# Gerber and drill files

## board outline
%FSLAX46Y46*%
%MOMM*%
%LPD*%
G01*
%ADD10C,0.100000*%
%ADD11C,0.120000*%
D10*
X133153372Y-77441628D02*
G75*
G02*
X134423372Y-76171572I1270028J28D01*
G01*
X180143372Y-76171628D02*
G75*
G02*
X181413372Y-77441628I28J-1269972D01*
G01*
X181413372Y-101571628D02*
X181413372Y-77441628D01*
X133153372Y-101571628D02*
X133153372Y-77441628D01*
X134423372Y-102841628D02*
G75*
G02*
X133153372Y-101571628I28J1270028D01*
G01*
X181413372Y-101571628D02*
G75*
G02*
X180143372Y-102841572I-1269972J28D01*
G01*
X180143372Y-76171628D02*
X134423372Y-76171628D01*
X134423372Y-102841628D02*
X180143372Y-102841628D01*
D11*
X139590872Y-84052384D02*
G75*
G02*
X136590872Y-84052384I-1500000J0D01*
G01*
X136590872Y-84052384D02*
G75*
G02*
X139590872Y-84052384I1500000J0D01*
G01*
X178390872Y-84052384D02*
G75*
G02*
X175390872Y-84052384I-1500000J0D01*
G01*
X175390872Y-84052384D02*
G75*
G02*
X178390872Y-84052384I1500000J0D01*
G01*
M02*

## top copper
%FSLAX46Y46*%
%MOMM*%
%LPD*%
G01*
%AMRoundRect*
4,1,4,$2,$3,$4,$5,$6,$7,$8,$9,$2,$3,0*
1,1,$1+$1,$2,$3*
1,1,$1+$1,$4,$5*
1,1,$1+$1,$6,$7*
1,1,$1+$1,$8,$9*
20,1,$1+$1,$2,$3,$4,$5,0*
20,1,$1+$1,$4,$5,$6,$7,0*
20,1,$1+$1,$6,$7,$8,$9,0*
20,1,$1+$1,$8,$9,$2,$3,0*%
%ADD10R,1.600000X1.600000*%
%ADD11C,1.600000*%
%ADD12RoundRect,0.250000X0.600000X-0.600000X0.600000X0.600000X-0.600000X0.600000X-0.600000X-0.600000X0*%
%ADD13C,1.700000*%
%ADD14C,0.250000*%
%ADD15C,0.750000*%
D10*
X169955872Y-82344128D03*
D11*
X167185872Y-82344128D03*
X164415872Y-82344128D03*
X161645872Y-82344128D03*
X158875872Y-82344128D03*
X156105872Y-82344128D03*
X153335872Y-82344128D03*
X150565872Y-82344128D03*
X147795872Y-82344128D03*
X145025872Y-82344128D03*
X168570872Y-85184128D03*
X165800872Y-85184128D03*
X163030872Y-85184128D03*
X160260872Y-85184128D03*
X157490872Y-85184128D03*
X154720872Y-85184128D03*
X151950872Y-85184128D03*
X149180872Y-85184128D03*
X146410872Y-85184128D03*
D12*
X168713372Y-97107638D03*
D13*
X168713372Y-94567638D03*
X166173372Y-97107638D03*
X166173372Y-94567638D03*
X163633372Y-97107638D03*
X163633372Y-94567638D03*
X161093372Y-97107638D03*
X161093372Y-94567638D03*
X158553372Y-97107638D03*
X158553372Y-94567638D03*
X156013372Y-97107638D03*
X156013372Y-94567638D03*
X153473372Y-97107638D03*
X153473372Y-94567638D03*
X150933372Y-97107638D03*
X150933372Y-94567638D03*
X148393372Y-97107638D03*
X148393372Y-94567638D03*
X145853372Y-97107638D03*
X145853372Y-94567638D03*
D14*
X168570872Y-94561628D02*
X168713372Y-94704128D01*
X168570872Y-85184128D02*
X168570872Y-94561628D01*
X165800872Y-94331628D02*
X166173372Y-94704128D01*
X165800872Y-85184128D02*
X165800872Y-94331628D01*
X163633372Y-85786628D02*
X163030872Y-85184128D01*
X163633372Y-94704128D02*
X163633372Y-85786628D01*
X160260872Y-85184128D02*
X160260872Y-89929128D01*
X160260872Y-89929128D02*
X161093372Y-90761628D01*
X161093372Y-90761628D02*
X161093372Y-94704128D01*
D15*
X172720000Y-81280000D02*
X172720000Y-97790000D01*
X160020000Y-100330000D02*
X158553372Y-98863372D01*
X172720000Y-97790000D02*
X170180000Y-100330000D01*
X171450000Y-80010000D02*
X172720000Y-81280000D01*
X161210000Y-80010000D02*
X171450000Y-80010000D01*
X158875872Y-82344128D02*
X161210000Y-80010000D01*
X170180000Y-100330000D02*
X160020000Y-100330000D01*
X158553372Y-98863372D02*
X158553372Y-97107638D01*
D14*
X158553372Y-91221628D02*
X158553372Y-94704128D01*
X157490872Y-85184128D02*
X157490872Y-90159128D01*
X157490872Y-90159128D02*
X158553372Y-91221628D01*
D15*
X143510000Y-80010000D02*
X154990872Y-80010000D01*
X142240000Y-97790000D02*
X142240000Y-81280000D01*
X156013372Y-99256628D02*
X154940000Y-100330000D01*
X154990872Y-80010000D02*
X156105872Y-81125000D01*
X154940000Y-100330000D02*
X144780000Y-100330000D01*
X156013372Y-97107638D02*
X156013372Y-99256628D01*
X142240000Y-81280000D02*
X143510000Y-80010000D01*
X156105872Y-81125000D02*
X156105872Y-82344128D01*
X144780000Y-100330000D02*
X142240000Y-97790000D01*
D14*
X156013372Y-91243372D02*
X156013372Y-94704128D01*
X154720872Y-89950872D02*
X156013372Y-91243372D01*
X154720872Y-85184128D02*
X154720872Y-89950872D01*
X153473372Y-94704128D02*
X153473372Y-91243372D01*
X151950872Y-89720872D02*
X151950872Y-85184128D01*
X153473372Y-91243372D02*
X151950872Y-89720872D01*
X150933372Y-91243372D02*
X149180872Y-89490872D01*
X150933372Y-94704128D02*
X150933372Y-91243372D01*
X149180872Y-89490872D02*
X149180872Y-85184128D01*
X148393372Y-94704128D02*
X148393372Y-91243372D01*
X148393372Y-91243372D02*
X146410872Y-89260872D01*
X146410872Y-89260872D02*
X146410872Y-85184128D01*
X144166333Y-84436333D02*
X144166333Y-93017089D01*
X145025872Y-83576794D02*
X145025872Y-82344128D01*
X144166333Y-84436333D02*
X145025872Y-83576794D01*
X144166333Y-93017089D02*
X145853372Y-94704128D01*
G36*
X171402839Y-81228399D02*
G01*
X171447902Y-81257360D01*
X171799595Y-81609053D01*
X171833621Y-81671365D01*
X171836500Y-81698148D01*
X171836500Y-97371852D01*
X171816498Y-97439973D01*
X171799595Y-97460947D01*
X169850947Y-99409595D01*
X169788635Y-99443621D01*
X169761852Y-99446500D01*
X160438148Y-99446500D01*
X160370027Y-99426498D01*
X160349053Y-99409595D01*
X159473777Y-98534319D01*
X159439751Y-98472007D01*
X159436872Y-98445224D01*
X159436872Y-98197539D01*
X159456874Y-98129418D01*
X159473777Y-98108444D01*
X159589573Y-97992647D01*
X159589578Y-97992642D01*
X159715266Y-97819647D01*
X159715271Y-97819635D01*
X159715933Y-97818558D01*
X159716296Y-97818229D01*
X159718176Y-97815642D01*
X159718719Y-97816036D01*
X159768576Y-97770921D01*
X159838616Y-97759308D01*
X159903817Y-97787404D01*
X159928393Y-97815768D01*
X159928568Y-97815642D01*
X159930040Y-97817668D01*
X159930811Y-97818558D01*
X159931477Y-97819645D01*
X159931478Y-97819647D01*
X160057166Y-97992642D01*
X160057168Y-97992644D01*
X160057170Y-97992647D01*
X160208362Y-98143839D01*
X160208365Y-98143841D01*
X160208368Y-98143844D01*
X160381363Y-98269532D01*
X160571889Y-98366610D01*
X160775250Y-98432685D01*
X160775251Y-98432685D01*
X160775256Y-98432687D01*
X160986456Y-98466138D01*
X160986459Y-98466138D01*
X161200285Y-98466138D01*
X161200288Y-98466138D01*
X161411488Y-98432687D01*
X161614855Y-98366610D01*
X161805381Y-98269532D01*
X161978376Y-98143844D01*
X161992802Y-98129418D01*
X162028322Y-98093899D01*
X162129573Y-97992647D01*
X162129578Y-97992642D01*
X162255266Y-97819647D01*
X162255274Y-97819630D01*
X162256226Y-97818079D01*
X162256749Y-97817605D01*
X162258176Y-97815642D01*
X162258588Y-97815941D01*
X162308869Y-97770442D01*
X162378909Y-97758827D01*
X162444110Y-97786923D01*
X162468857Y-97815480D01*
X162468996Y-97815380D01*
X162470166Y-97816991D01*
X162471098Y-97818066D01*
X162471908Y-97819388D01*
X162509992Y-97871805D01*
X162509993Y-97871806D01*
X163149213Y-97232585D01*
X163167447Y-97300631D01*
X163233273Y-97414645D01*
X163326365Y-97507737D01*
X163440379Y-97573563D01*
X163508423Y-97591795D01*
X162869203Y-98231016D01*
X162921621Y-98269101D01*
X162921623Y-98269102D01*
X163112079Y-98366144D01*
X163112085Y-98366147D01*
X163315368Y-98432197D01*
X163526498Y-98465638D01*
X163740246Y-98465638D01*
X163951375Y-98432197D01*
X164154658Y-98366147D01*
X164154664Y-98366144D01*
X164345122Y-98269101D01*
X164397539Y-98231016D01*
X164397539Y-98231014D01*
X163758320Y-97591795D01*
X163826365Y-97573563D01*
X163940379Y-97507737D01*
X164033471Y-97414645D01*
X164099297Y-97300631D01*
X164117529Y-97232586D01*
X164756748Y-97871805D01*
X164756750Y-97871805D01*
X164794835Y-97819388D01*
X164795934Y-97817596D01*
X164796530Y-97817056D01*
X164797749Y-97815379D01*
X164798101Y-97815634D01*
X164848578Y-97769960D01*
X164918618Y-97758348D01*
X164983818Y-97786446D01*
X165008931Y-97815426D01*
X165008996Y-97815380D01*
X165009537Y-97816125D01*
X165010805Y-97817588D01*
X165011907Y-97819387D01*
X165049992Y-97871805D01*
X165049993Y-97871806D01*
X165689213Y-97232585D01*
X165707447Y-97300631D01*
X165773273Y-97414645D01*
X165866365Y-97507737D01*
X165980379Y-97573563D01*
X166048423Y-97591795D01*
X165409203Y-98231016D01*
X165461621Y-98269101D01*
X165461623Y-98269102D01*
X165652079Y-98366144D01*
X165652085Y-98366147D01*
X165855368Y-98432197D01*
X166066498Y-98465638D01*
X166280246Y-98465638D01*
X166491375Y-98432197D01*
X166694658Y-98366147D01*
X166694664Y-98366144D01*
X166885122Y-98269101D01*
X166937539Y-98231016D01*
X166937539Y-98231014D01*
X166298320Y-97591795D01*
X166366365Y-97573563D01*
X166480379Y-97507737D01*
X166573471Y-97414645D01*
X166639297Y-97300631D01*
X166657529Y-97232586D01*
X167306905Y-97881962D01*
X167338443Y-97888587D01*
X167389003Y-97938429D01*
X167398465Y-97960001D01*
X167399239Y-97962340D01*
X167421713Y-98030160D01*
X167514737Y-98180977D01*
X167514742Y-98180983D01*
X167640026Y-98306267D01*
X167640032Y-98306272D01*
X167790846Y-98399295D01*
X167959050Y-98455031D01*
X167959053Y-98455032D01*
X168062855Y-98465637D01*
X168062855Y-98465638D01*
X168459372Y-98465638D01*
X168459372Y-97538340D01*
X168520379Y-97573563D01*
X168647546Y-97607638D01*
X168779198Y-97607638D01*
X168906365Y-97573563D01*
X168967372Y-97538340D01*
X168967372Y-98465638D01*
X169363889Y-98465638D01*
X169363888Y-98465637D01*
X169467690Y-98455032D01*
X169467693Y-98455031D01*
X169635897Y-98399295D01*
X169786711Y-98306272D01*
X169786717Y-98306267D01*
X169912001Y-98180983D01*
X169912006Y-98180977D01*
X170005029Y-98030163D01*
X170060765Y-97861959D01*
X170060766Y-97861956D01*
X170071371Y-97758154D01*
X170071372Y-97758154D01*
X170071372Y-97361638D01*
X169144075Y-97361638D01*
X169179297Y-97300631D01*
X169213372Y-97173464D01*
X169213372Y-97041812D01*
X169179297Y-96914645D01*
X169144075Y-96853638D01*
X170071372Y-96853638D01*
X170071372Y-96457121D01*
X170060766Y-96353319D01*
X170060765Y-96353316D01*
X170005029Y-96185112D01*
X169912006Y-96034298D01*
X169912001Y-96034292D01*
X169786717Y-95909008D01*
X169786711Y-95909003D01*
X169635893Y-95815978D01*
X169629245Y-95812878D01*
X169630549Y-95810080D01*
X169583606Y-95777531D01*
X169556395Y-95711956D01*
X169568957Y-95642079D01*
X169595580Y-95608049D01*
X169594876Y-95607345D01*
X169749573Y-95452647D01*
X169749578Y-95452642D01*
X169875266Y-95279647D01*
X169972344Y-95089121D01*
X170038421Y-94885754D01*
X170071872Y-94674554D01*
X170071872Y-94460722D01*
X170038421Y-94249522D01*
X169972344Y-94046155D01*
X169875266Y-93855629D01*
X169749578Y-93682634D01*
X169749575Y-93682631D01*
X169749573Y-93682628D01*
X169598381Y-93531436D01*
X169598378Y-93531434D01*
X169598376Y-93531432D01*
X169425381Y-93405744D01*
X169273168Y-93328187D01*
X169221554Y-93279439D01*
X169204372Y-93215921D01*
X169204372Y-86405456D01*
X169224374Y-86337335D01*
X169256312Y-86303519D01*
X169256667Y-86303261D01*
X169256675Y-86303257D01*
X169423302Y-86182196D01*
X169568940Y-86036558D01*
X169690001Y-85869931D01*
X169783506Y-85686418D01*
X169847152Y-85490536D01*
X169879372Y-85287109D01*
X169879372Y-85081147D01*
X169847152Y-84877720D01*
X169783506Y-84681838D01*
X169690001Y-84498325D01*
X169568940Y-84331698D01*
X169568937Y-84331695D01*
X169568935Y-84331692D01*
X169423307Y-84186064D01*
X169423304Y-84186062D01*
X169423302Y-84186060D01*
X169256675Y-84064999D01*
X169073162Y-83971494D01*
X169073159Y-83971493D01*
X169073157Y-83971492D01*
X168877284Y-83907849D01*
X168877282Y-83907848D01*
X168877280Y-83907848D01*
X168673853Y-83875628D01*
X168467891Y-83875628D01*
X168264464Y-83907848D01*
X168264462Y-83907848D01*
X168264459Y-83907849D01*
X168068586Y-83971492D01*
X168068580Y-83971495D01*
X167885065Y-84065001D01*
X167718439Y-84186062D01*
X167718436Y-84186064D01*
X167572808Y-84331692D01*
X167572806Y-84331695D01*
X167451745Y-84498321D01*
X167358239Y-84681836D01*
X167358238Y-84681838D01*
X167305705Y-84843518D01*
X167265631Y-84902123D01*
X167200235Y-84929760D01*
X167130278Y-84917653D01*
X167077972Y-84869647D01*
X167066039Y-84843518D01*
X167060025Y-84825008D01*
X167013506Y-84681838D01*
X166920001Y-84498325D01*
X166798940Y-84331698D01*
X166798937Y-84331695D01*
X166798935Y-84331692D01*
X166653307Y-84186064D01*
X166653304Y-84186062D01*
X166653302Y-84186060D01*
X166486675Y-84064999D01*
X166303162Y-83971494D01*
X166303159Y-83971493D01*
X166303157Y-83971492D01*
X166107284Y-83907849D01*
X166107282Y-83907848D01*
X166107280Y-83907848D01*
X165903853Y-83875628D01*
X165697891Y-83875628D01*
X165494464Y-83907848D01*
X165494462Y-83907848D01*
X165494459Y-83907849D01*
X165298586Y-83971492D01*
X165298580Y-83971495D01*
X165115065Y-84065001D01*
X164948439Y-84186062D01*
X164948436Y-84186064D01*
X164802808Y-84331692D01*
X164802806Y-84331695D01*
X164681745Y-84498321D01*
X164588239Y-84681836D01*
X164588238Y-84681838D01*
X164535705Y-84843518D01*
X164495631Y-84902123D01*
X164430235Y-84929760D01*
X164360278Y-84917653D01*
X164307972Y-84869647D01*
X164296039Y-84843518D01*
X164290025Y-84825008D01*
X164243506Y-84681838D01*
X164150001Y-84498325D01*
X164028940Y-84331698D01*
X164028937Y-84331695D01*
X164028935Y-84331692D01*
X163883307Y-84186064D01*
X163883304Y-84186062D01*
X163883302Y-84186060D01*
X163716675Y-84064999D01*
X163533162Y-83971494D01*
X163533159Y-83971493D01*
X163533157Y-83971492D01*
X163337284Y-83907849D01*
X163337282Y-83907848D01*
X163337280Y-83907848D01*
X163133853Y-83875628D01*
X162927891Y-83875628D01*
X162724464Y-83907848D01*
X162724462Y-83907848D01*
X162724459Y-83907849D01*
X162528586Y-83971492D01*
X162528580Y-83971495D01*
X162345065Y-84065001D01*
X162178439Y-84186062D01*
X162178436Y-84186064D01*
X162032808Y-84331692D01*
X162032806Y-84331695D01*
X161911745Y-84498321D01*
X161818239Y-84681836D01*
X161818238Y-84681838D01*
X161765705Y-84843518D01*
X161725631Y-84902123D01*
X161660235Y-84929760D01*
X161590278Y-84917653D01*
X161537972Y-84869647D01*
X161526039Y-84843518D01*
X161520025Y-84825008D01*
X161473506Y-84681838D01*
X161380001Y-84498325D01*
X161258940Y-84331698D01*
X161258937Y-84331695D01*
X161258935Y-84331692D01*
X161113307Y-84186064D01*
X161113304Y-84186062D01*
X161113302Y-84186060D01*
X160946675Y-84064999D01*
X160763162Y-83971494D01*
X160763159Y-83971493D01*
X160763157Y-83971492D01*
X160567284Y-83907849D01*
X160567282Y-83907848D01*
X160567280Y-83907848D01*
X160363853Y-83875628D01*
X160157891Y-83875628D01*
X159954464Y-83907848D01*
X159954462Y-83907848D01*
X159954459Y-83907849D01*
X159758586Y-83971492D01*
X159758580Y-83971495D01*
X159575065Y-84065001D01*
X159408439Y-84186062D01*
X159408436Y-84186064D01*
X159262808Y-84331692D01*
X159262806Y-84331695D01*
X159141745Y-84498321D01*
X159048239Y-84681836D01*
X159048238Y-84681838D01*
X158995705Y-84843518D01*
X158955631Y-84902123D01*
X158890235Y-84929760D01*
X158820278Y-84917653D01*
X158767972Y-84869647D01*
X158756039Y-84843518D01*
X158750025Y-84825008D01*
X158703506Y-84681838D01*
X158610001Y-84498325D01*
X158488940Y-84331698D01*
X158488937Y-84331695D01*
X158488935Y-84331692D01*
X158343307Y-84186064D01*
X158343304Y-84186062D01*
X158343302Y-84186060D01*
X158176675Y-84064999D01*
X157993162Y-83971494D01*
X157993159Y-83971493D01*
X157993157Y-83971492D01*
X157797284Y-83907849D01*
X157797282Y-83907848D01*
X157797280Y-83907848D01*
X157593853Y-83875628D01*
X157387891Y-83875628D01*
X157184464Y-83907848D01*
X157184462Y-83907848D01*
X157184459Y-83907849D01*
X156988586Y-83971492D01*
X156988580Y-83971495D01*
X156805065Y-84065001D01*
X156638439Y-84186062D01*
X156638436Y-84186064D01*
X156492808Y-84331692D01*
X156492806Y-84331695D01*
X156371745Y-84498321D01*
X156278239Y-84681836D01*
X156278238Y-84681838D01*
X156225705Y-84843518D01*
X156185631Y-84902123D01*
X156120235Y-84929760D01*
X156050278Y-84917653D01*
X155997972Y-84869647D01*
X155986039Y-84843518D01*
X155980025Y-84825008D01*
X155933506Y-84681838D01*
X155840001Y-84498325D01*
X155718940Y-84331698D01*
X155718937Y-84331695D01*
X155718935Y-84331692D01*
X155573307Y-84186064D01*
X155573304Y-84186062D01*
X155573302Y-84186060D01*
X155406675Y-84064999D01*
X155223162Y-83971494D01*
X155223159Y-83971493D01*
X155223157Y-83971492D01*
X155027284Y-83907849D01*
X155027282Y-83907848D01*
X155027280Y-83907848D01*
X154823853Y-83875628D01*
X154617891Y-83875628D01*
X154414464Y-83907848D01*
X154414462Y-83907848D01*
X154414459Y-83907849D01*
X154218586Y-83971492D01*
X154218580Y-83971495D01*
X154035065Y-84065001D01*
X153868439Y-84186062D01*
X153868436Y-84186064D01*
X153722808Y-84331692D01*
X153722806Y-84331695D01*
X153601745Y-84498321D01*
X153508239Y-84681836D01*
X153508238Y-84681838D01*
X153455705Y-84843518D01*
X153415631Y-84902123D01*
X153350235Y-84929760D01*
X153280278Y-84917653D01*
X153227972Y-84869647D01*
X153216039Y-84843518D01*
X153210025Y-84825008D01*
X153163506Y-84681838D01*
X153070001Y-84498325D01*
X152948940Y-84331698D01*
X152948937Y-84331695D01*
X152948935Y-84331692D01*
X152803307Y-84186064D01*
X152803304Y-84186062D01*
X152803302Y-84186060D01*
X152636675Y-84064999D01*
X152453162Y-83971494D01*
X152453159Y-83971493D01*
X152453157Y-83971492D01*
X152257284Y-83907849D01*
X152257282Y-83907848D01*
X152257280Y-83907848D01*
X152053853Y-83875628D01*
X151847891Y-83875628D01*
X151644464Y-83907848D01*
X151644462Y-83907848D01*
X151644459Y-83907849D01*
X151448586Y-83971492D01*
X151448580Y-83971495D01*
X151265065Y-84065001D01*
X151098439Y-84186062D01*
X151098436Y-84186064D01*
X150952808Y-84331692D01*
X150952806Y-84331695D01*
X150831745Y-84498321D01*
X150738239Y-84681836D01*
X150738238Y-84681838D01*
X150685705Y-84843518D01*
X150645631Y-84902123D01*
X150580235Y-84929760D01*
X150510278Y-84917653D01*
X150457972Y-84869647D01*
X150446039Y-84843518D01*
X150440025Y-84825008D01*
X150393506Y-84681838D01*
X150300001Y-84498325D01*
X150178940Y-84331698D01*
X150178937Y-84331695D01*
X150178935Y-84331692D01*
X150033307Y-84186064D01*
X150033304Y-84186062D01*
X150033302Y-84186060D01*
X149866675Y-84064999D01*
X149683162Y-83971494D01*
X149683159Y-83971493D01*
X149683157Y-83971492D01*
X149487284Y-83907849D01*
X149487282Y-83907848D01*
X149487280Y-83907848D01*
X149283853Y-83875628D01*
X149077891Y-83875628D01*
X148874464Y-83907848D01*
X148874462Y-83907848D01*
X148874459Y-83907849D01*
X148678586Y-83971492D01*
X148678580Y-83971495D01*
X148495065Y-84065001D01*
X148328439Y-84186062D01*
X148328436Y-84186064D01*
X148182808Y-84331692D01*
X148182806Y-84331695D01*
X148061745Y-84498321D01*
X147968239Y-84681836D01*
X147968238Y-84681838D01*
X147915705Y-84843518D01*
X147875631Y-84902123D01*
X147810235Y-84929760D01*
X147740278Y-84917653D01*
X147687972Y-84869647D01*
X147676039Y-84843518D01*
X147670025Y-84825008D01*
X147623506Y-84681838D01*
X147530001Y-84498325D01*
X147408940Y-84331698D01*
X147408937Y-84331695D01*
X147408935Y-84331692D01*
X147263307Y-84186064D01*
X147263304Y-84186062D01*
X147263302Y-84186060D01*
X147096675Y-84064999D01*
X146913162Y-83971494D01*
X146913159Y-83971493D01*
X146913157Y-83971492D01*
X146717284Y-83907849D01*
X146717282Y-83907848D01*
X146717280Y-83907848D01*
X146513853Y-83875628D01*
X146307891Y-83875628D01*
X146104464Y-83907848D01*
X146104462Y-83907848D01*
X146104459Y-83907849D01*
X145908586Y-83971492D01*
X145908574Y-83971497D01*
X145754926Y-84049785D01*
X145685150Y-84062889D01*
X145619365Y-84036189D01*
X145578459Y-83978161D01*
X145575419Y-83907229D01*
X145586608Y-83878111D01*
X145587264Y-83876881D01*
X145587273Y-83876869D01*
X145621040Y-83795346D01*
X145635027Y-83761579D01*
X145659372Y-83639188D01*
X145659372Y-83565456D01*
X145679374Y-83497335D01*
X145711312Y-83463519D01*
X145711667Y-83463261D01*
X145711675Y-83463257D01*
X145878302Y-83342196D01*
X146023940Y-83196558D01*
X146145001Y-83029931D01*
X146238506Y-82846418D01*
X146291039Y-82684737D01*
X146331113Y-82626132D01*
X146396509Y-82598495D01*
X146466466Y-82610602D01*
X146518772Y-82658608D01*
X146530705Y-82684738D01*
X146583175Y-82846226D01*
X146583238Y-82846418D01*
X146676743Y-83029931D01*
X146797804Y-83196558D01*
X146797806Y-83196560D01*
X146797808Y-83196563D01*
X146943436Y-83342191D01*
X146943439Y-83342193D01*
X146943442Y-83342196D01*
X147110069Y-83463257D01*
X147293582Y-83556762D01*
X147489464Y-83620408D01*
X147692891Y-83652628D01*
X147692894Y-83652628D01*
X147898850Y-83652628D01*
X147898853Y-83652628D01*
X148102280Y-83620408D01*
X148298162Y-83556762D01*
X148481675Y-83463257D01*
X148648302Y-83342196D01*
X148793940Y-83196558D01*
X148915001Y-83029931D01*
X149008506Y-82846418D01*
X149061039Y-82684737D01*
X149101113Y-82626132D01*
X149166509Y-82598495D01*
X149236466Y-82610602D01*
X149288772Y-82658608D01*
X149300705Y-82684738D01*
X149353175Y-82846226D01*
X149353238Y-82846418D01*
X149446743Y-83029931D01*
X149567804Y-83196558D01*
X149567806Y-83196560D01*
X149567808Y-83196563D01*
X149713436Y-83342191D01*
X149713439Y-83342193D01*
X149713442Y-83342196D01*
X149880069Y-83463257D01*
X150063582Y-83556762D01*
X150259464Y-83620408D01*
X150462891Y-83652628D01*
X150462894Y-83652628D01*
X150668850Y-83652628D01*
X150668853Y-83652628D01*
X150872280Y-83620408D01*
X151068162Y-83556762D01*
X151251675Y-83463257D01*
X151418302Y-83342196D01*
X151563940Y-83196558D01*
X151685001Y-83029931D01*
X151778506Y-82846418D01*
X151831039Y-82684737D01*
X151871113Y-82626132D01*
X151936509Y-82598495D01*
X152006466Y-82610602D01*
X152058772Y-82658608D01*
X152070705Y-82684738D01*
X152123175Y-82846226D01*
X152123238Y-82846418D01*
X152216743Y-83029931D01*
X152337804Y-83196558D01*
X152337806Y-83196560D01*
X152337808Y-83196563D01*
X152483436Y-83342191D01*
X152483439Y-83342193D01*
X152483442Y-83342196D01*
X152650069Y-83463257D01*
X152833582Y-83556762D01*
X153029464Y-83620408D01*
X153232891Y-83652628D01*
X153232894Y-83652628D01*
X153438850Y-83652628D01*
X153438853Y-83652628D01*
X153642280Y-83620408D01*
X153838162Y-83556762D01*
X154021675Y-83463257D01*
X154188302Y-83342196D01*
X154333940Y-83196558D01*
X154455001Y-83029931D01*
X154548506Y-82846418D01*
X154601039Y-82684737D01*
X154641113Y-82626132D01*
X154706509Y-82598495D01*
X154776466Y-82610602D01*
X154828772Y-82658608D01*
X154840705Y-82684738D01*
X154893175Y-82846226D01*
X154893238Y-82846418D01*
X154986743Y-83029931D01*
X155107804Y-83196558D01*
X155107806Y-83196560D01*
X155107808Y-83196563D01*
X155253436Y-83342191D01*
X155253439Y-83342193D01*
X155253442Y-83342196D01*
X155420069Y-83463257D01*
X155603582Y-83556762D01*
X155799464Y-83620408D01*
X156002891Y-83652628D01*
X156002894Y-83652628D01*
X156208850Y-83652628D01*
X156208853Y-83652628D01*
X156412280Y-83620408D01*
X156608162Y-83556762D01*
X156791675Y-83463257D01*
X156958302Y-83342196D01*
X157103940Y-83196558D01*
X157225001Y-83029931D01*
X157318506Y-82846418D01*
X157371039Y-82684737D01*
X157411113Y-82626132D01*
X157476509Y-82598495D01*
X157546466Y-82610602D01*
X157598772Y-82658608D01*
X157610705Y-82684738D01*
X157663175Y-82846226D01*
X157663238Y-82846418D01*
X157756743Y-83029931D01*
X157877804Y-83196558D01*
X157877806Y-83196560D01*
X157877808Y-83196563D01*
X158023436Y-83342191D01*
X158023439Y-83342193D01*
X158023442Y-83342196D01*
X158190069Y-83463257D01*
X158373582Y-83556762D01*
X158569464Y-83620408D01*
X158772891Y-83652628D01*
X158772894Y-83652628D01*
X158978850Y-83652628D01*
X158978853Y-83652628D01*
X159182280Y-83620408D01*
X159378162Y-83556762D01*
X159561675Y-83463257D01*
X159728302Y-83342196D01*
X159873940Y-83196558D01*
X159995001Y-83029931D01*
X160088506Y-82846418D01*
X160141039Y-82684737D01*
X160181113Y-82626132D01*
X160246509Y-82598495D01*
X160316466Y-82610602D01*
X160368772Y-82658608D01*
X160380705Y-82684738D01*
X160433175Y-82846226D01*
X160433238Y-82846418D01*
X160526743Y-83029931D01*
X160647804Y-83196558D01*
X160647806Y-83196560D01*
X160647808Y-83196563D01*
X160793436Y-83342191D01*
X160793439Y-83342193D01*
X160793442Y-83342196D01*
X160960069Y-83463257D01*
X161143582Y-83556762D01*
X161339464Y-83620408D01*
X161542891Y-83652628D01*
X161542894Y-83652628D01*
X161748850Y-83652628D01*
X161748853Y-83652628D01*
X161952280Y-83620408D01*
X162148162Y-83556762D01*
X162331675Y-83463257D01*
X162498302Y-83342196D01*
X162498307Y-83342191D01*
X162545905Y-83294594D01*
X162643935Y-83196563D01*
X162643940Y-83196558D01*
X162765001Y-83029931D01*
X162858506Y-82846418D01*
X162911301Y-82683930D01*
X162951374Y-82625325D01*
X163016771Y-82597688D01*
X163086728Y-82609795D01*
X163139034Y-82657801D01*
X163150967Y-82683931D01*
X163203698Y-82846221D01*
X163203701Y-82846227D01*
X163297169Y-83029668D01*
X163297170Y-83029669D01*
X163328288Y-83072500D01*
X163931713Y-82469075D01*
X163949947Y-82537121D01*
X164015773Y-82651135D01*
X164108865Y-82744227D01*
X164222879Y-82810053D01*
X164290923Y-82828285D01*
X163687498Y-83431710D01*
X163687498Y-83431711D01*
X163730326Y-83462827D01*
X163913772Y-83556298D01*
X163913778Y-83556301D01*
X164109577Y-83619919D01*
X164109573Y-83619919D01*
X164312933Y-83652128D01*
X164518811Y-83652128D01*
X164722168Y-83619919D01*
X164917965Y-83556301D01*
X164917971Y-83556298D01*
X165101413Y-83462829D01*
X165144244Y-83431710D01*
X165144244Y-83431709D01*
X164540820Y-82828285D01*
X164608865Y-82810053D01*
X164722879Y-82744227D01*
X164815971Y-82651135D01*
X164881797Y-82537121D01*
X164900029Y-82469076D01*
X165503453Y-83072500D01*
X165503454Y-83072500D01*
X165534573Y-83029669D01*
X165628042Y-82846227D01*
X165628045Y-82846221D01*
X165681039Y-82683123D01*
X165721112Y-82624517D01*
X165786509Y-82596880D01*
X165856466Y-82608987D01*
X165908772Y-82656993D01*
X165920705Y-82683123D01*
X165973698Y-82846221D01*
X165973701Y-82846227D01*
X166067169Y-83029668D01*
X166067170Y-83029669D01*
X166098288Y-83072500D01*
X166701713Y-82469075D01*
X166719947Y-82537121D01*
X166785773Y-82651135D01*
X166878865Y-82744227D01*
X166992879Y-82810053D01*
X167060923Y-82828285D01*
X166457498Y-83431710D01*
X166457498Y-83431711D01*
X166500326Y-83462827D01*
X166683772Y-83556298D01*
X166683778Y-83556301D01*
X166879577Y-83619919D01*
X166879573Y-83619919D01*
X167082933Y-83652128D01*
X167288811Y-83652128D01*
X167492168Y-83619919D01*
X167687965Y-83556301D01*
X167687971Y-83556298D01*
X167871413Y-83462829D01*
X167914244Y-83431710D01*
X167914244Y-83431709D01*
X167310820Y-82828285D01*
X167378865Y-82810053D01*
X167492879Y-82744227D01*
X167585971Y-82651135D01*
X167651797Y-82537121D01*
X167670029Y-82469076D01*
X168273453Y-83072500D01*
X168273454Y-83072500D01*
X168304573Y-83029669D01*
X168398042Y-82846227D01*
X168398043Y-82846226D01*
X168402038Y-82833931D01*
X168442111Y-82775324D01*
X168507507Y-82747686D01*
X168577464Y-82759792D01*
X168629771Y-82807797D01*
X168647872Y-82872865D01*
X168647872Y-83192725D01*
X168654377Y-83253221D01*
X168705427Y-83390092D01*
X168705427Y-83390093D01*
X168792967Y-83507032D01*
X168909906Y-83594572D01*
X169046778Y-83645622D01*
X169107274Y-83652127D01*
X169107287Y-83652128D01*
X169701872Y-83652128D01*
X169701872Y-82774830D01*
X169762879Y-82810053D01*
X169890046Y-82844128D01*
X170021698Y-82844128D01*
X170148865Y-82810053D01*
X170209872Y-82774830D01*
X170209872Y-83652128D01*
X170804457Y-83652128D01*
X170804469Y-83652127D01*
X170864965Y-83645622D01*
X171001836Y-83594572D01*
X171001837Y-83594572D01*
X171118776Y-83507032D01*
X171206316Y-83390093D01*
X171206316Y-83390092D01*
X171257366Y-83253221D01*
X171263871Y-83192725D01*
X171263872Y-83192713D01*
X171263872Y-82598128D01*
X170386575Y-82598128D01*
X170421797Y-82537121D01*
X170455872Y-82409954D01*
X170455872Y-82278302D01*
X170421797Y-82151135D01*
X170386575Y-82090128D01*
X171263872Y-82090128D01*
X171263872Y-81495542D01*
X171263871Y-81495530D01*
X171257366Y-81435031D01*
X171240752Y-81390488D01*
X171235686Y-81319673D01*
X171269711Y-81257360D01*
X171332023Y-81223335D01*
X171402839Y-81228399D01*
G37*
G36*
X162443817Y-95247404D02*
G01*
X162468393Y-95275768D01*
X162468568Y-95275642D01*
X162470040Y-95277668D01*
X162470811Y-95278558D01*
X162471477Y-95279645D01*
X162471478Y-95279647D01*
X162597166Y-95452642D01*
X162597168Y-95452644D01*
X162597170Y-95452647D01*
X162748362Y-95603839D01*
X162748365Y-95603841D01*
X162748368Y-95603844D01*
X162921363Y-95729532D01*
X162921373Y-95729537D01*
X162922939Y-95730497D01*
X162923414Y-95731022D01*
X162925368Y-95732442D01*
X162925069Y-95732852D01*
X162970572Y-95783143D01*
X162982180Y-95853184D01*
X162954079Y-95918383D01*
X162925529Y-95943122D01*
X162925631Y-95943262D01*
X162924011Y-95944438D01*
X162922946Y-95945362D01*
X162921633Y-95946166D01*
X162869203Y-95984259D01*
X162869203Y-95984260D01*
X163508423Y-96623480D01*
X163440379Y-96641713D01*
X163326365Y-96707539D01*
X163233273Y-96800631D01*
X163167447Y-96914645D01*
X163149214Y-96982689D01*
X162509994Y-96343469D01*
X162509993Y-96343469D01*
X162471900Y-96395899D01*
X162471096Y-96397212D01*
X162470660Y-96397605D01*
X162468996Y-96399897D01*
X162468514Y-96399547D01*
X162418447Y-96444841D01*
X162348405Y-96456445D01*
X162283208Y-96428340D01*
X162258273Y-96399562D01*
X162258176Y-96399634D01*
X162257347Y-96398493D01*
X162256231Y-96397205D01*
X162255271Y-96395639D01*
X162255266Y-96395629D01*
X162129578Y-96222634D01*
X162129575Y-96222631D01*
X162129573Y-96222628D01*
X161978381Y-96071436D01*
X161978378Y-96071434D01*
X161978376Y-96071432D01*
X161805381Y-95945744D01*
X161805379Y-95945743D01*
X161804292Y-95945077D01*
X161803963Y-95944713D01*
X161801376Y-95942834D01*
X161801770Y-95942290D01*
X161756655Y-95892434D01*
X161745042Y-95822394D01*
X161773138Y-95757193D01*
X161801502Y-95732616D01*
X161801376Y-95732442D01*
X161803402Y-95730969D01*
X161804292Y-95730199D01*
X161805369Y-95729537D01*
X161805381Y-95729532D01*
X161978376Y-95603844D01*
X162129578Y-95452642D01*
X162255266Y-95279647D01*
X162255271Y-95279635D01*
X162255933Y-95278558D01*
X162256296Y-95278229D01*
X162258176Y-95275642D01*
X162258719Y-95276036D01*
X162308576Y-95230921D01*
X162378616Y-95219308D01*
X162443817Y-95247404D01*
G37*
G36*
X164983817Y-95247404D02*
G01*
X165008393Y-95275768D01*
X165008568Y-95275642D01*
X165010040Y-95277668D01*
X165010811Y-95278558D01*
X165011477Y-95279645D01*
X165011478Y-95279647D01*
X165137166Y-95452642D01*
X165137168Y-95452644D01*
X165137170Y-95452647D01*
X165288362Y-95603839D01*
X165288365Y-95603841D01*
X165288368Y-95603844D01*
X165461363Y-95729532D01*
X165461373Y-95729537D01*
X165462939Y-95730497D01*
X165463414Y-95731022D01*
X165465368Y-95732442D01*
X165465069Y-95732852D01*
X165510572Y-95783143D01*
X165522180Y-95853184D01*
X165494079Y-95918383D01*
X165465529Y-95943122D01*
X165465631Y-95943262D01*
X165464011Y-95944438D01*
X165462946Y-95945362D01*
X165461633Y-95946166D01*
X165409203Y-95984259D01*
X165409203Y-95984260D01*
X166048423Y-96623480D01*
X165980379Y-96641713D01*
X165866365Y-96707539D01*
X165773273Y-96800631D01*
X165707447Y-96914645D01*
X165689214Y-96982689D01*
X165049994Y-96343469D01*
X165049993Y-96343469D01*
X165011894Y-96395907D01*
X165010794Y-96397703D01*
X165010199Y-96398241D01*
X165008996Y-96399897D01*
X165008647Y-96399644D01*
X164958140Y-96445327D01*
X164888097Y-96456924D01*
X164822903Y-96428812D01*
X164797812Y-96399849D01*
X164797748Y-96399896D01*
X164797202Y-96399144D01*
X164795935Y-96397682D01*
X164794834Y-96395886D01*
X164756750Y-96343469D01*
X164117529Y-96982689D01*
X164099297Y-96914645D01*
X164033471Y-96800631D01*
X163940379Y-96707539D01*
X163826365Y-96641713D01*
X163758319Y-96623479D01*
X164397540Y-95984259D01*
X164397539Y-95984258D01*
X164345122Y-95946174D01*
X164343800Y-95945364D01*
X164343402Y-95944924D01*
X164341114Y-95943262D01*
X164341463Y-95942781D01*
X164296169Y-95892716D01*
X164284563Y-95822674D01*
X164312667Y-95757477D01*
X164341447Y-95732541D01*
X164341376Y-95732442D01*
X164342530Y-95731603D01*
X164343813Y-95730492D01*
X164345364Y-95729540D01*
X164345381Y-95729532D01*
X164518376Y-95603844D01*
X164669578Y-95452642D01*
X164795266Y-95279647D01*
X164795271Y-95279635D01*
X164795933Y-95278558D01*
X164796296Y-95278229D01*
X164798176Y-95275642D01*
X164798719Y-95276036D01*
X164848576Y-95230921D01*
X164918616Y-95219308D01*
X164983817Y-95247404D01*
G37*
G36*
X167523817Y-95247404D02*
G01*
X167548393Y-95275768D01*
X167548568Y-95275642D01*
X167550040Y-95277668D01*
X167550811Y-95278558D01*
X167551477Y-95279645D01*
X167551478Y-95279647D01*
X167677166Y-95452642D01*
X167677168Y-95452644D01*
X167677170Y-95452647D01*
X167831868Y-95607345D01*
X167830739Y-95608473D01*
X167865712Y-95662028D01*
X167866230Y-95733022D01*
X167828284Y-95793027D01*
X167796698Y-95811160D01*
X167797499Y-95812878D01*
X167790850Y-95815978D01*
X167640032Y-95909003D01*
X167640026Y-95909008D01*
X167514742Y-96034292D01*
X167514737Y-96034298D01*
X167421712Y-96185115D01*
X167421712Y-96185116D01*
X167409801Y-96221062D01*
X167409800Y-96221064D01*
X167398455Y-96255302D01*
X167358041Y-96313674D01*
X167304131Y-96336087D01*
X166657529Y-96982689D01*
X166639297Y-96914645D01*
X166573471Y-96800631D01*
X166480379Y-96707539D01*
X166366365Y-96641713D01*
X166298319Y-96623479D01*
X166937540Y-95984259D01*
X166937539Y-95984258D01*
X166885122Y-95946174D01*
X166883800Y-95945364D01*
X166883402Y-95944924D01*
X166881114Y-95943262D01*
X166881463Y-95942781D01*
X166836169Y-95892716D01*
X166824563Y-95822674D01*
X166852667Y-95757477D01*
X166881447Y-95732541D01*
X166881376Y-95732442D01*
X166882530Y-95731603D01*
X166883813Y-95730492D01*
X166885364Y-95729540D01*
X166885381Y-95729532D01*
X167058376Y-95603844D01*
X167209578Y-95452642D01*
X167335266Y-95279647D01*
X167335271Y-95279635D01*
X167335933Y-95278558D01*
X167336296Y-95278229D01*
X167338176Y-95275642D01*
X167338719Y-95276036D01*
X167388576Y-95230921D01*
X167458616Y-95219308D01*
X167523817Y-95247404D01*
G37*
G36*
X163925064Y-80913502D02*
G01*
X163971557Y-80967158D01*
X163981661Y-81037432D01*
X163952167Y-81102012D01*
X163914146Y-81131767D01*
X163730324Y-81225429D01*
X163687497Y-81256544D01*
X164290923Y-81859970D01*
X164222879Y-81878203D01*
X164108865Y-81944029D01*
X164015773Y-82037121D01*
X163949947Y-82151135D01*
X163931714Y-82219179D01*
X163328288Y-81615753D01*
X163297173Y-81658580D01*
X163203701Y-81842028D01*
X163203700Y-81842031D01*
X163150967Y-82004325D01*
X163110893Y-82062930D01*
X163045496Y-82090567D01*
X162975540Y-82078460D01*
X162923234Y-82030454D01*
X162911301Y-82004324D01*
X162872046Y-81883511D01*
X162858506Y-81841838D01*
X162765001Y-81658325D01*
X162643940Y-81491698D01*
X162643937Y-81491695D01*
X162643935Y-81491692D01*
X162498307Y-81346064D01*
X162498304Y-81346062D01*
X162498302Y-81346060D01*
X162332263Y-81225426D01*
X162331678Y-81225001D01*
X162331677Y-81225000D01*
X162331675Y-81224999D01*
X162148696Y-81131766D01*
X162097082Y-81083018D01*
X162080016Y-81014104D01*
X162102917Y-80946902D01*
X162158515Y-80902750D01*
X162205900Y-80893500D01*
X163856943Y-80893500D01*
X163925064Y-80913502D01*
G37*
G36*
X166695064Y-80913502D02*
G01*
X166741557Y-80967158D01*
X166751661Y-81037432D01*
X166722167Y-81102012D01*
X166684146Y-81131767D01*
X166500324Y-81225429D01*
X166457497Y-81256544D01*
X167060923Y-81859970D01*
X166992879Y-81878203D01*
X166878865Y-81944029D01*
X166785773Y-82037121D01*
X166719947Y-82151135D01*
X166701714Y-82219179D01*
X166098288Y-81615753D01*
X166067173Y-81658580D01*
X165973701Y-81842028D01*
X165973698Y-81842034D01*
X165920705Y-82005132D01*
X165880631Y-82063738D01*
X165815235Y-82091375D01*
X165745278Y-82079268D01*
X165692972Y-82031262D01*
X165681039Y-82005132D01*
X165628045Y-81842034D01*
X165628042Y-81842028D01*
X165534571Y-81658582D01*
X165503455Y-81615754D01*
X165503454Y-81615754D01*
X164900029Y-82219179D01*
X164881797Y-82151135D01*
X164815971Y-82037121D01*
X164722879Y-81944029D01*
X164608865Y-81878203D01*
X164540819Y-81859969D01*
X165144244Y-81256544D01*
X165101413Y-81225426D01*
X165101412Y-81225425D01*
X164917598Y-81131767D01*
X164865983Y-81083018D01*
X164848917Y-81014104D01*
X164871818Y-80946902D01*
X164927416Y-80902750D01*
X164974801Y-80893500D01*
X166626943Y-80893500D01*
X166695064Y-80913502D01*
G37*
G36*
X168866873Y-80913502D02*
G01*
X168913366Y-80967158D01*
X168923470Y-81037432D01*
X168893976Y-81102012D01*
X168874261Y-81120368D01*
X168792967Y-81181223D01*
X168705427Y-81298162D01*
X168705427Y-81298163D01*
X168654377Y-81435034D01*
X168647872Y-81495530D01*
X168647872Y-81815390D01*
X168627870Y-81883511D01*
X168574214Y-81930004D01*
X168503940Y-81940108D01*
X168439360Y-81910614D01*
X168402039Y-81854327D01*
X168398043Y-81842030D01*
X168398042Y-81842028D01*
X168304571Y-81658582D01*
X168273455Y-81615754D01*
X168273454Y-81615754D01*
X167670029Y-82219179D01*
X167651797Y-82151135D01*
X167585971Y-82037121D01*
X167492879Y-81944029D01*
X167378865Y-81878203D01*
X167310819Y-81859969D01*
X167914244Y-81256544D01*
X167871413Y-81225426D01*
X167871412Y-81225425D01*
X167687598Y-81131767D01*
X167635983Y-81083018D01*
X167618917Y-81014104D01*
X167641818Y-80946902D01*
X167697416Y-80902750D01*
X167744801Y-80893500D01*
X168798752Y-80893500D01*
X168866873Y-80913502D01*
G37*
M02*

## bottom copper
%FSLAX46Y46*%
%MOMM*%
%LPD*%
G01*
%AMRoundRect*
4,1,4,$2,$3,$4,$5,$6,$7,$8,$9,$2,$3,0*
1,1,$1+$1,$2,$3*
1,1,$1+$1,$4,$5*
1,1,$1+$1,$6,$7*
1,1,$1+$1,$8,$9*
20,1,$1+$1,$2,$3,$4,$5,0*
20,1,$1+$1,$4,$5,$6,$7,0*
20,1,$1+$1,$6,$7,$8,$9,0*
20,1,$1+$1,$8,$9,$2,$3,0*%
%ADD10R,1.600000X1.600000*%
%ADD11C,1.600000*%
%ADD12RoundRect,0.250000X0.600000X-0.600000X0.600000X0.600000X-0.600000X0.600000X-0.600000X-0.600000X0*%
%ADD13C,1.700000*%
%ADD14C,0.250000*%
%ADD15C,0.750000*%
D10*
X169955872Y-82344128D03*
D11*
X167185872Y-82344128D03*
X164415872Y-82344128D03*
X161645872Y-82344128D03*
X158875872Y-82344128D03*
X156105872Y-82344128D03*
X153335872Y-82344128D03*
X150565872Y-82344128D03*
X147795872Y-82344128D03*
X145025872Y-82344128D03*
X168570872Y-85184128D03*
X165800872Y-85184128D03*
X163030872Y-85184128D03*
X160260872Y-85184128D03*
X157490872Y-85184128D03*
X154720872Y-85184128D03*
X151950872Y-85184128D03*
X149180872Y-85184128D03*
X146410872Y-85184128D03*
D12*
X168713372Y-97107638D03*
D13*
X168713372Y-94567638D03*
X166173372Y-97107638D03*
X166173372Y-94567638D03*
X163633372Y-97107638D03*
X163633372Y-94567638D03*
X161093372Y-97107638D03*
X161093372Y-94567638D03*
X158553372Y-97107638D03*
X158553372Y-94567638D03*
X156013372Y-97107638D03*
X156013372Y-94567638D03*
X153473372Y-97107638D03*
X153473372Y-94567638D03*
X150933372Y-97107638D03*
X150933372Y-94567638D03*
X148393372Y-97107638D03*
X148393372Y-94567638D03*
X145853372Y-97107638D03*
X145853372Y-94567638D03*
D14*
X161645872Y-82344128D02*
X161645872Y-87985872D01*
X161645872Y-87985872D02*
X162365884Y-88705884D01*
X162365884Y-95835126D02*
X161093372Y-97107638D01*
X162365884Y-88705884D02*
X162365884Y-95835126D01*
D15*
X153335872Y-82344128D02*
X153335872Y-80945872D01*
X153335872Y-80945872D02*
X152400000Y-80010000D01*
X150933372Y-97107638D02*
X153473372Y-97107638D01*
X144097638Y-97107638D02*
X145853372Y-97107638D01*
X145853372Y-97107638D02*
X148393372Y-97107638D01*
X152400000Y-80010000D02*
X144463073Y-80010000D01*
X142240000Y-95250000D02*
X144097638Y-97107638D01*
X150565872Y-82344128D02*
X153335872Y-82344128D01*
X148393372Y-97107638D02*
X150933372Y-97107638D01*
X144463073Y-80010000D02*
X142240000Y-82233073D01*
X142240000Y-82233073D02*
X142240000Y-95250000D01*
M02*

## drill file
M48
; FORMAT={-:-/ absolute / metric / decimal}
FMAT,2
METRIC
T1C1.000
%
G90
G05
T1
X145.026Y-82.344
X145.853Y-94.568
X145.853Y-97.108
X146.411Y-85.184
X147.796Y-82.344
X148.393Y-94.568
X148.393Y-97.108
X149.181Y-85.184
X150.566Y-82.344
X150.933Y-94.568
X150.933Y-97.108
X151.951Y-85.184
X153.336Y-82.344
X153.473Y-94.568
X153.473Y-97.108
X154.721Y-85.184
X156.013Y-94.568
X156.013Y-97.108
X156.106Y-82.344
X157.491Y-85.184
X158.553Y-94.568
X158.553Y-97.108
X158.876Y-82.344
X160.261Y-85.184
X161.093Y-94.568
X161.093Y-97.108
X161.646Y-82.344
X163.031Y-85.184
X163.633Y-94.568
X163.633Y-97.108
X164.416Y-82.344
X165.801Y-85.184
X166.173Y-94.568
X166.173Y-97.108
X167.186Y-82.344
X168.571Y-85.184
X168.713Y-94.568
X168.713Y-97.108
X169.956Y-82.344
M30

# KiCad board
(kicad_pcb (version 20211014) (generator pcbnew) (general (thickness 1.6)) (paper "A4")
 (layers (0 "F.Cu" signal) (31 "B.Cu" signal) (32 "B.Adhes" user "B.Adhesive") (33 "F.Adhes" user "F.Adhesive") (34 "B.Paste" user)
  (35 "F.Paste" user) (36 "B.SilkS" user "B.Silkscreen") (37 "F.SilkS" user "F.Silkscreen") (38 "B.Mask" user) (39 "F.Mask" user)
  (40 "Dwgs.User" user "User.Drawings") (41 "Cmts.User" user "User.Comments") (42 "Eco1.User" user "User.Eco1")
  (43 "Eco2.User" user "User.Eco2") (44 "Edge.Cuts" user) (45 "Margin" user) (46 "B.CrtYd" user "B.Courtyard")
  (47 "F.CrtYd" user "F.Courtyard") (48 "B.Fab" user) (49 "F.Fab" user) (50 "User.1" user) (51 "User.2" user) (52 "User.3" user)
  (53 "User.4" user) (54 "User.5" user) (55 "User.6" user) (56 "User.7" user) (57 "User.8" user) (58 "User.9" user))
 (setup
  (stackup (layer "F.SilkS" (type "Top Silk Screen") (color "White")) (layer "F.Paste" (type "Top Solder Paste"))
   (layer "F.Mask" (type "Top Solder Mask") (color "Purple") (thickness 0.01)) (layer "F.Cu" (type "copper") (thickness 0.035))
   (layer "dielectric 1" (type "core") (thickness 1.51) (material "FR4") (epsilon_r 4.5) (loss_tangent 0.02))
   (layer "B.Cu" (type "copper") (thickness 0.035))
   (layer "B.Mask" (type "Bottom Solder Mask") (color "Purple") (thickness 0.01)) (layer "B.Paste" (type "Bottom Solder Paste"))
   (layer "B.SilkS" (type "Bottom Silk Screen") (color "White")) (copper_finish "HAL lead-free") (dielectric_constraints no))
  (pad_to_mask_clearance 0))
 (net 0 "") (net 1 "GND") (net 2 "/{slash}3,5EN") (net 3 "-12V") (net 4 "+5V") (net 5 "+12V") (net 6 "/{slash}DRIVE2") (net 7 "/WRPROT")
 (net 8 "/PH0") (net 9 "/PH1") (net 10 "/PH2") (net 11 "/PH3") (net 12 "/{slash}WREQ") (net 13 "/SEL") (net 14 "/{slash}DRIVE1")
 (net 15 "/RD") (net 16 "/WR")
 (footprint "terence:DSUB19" (layer "F.Cu") (at 157.490872 72.184128)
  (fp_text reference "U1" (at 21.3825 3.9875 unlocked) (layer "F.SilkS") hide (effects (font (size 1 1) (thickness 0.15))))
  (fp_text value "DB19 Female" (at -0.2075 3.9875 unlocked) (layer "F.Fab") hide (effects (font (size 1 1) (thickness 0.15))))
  (fp_circle (center -19.4 11.868256) (end -17.9 11.868256) (layer "Edge.Cuts") (width 0.12) (fill none))
  (fp_circle (center 19.4 11.868256) (end 20.9 11.868256) (layer "Edge.Cuts") (width 0.12) (fill none))
  (pad "1" thru_hole rect (at 12.465 10.16) (size 1.6 1.6) (drill 1) (layers *.Cu *.Mask) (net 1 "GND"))
  (pad "2" thru_hole circle (at 9.695 10.16) (size 1.6 1.6) (drill 1) (layers *.Cu *.Mask) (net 1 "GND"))
  (pad "3" thru_hole circle (at 6.925 10.16) (size 1.6 1.6) (drill 1) (layers *.Cu *.Mask) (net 1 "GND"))
  (pad "4" thru_hole circle (at 4.155 10.16) (size 1.6 1.6) (drill 1) (layers *.Cu *.Mask) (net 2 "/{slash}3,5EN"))
  (pad "5" thru_hole circle (at 1.385 10.16) (size 1.6 1.6) (drill 1) (layers *.Cu *.Mask) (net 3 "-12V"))
  (pad "6" thru_hole circle (at -1.385 10.16) (size 1.6 1.6) (drill 1) (layers *.Cu *.Mask) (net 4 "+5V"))
  (pad "7" thru_hole circle (at -4.155 10.16) (size 1.6 1.6) (drill 1) (layers *.Cu *.Mask) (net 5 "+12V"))
  (pad "8" thru_hole circle (at -6.925 10.16) (size 1.6 1.6) (drill 1) (layers *.Cu *.Mask) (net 5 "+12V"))
  (pad "9" thru_hole circle (at -9.695 10.16) (size 1.6 1.6) (drill 1) (layers *.Cu *.Mask) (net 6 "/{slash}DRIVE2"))
  (pad "10" thru_hole circle (at -12.465 10.16) (size 1.6 1.6) (drill 1) (layers *.Cu *.Mask) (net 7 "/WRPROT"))
  (pad "11" thru_hole circle (at 11.08 13) (size 1.6 1.6) (drill 1) (layers *.Cu *.Mask) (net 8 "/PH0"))
  (pad "12" thru_hole circle (at 8.31 13) (size 1.6 1.6) (drill 1) (layers *.Cu *.Mask) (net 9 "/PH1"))
  (pad "13" thru_hole circle (at 5.54 13) (size 1.6 1.6) (drill 1) (layers *.Cu *.Mask) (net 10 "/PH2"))
  (pad "14" thru_hole circle (at 2.77 13) (size 1.6 1.6) (drill 1) (layers *.Cu *.Mask) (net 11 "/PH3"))
  (pad "15" thru_hole circle (at 0 13) (size 1.6 1.6) (drill 1) (layers *.Cu *.Mask) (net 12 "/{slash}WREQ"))
  (pad "16" thru_hole circle (at -2.77 13) (size 1.6 1.6) (drill 1) (layers *.Cu *.Mask) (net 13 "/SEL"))
  (pad "17" thru_hole circle (at -5.54 13) (size 1.6 1.6) (drill 1) (layers *.Cu *.Mask) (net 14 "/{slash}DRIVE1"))
  (pad "18" thru_hole circle (at -8.31 13) (size 1.6 1.6) (drill 1) (layers *.Cu *.Mask) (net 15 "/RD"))
  (pad "19" thru_hole circle (at -11.08 13) (size 1.6 1.6) (drill 1) (layers *.Cu *.Mask) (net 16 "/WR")))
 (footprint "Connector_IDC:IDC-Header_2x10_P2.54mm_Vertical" (layer "B.Cu") (at 168.713372 97.107638 90)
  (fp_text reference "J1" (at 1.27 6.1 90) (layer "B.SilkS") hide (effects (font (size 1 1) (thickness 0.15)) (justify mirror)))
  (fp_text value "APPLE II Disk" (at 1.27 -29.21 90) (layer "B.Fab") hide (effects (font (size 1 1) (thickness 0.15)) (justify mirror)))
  (pad "1" thru_hole roundrect (at 0 0 90) (size 1.7 1.7) (drill 1) (layers *.Cu *.Mask) (roundrect_rratio 0.1470588235) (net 1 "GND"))
  (pad "2" thru_hole circle (at 2.54 0 90) (size 1.7 1.7) (drill 1) (layers *.Cu *.Mask) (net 8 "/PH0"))
  (pad "3" thru_hole circle (at 0 -2.54 90) (size 1.7 1.7) (drill 1) (layers *.Cu *.Mask) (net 1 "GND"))
  (pad "4" thru_hole circle (at 2.54 -2.54 90) (size 1.7 1.7) (drill 1) (layers *.Cu *.Mask) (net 9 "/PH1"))
  (pad "5" thru_hole circle (at 0 -5.08 90) (size 1.7 1.7) (drill 1) (layers *.Cu *.Mask) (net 1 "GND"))
  (pad "6" thru_hole circle (at 2.54 -5.08 90) (size 1.7 1.7) (drill 1) (layers *.Cu *.Mask) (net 10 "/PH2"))
  (pad "7" thru_hole circle (at 0 -7.62 90) (size 1.7 1.7) (drill 1) (layers *.Cu *.Mask) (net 2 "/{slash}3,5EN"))
  (pad "8" thru_hole circle (at 2.54 -7.62 90) (size 1.7 1.7) (drill 1) (layers *.Cu *.Mask) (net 11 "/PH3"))
  (pad "9" thru_hole circle (at 0 -10.16 90) (size 1.7 1.7) (drill 1) (layers *.Cu *.Mask) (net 3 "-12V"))
  (pad "10" thru_hole circle (at 2.54 -10.16 90) (size 1.7 1.7) (drill 1) (layers *.Cu *.Mask) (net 12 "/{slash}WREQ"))
  (pad "11" thru_hole circle (at 0 -12.7 90) (size 1.7 1.7) (drill 1) (layers *.Cu *.Mask) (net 4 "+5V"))
  (pad "12" thru_hole circle (at 2.54 -12.7 90) (size 1.7 1.7) (drill 1) (layers *.Cu *.Mask) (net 13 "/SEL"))
  (pad "13" thru_hole circle (at 0 -15.24 90) (size 1.7 1.7) (drill 1) (layers *.Cu *.Mask) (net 5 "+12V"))
  (pad "14" thru_hole circle (at 2.54 -15.24 90) (size 1.7 1.7) (drill 1) (layers *.Cu *.Mask) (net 14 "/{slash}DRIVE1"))
  (pad "15" thru_hole circle (at 0 -17.78 90) (size 1.7 1.7) (drill 1) (layers *.Cu *.Mask) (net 5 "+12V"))
  (pad "16" thru_hole circle (at 2.54 -17.78 90) (size 1.7 1.7) (drill 1) (layers *.Cu *.Mask) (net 15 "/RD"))
  (pad "17" thru_hole circle (at 0 -20.32 90) (size 1.7 1.7) (drill 1) (layers *.Cu *.Mask) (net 5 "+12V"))
  (pad "18" thru_hole circle (at 2.54 -20.32 90) (size 1.7 1.7) (drill 1) (layers *.Cu *.Mask) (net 16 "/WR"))
  (pad "19" thru_hole circle (at 0 -22.86 90) (size 1.7 1.7) (drill 1) (layers *.Cu *.Mask) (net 5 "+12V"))
  (pad "20" thru_hole circle (at 2.54 -22.86 90) (size 1.7 1.7) (drill 1) (layers *.Cu *.Mask) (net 7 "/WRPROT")))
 (gr_arc (start 133.153372 77.441628) (mid 133.525346 76.543602) (end 134.423372 76.171628) (layer "Edge.Cuts") (width 0.1))
 (gr_arc (start 180.143372 76.171628) (mid 181.041398 76.543602) (end 181.413372 77.441628) (layer "Edge.Cuts") (width 0.1))
 (gr_line (start 181.413372 101.571628) (end 181.413372 77.441628) (layer "Edge.Cuts") (width 0.1))
 (gr_line (start 133.153372 101.571628) (end 133.153372 77.441628) (layer "Edge.Cuts") (width 0.1))
 (gr_arc (start 134.423372 102.841628) (mid 133.525346 102.469654) (end 133.153372 101.571628) (layer "Edge.Cuts") (width 0.1))
 (gr_arc (start 181.413372 101.571628) (mid 181.041398 102.469654) (end 180.143372 102.841628) (layer "Edge.Cuts") (width 0.1))
 (gr_line (start 180.143372 76.171628) (end 134.423372 76.171628) (layer "Edge.Cuts") (width 0.1))
 (gr_line (start 134.423372 102.841628) (end 180.143372 102.841628) (layer "Edge.Cuts") (width 0.1))
 (segment (start 168.570872 94.561628) (end 168.713372 94.704128) (width 0.25) (layer "F.Cu") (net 8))
 (segment (start 168.570872 85.184128) (end 168.570872 94.561628) (width 0.25) (layer "F.Cu") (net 8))
 (segment (start 165.800872 94.331628) (end 166.173372 94.704128) (width 0.25) (layer "F.Cu") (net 9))
 (segment (start 165.800872 85.184128) (end 165.800872 94.331628) (width 0.25) (layer "F.Cu") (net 9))
 (segment (start 163.633372 85.786628) (end 163.030872 85.184128) (width 0.25) (layer "F.Cu") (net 10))
 (segment (start 163.633372 94.704128) (end 163.633372 85.786628) (width 0.25) (layer "F.Cu") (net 10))
 (segment (start 161.645872 82.344128) (end 161.645872 87.985872) (width 0.25) (layer "B.Cu") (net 2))
 (segment (start 161.645872 87.985872) (end 162.365884 88.705884) (width 0.25) (layer "B.Cu") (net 2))
 (segment (start 162.365884 95.835126) (end 161.093372 97.107638) (width 0.25) (layer "B.Cu") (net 2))
 (segment (start 162.365884 88.705884) (end 162.365884 95.835126) (width 0.25) (layer "B.Cu") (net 2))
 (segment (start 160.260872 85.184128) (end 160.260872 89.929128) (width 0.25) (layer "F.Cu") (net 11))
 (segment (start 160.260872 89.929128) (end 161.093372 90.761628) (width 0.25) (layer "F.Cu") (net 11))
 (segment (start 161.093372 90.761628) (end 161.093372 94.704128) (width 0.25) (layer "F.Cu") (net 11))
 (segment (start 172.72 81.28) (end 172.72 97.79) (width 0.75) (layer "F.Cu") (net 3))
 (segment (start 160.02 100.33) (end 158.553372 98.863372) (width 0.75) (layer "F.Cu") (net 3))
 (segment (start 172.72 97.79) (end 170.18 100.33) (width 0.75) (layer "F.Cu") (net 3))
 (segment (start 171.45 80.01) (end 172.72 81.28) (width 0.75) (layer "F.Cu") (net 3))
 (segment (start 161.21 80.01) (end 171.45 80.01) (width 0.75) (layer "F.Cu") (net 3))
 (segment (start 158.875872 82.344128) (end 161.21 80.01) (width 0.75) (layer "F.Cu") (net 3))
 (segment (start 170.18 100.33) (end 160.02 100.33) (width 0.75) (layer "F.Cu") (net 3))
 (segment (start 158.553372 98.863372) (end 158.553372 97.107638) (width 0.75) (layer "F.Cu") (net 3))
 (segment (start 158.553372 91.221628) (end 158.553372 94.704128) (width 0.25) (layer "F.Cu") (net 12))
 (segment (start 157.490872 85.184128) (end 157.490872 90.159128) (width 0.25) (layer "F.Cu") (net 12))
 (segment (start 157.490872 90.159128) (end 158.553372 91.221628) (width 0.25) (layer "F.Cu") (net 12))
 (segment (start 143.51 80.01) (end 154.990872 80.01) (width 0.75) (layer "F.Cu") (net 4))
 (segment (start 142.24 97.79) (end 142.24 81.28) (width 0.75) (layer "F.Cu") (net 4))
 (segment (start 156.013372 99.256628) (end 154.94 100.33) (width 0.75) (layer "F.Cu") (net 4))
 (segment (start 154.990872 80.01) (end 156.105872 81.125) (width 0.75) (layer "F.Cu") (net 4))
 (segment (start 154.94 100.33) (end 144.78 100.33) (width 0.75) (layer "F.Cu") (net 4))
 (segment (start 156.013372 97.107638) (end 156.013372 99.256628) (width 0.75) (layer "F.Cu") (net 4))
 (segment (start 142.24 81.28) (end 143.51 80.01) (width 0.75) (layer "F.Cu") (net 4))
 (segment (start 156.105872 81.125) (end 156.105872 82.344128) (width 0.75) (layer "F.Cu") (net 4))
 (segment (start 144.78 100.33) (end 142.24 97.79) (width 0.75) (layer "F.Cu") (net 4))
 (segment (start 156.013372 91.243372) (end 156.013372 94.704128) (width 0.25) (layer "F.Cu") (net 13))
 (segment (start 154.720872 89.950872) (end 156.013372 91.243372) (width 0.25) (layer "F.Cu") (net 13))
 (segment (start 154.720872 85.184128) (end 154.720872 89.950872) (width 0.25) (layer "F.Cu") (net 13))
 (segment (start 153.335872 82.344128) (end 153.335872 80.945872) (width 0.75) (layer "B.Cu") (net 5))
 (segment (start 153.335872 80.945872) (end 152.4 80.01) (width 0.75) (layer "B.Cu") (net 5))
 (segment (start 150.933372 97.107638) (end 153.473372 97.107638) (width 0.75) (layer "B.Cu") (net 5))
 (segment (start 144.097638 97.107638) (end 145.853372 97.107638) (width 0.75) (layer "B.Cu") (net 5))
 (segment (start 145.853372 97.107638) (end 148.393372 97.107638) (width 0.75) (layer "B.Cu") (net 5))
 (segment (start 152.4 80.01) (end 144.463073 80.01) (width 0.75) (layer "B.Cu") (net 5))
 (segment (start 142.24 95.25) (end 144.097638 97.107638) (width 0.75) (layer "B.Cu") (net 5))
 (segment (start 150.565872 82.344128) (end 153.335872 82.344128) (width 0.75) (layer "B.Cu") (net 5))
 (segment (start 148.393372 97.107638) (end 150.933372 97.107638) (width 0.75) (layer "B.Cu") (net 5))
 (segment (start 144.463073 80.01) (end 142.24 82.233073) (width 0.75) (layer "B.Cu") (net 5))
 (segment (start 142.24 82.233073) (end 142.24 95.25) (width 0.75) (layer "B.Cu") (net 5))
 (segment (start 153.473372 94.704128) (end 153.473372 91.243372) (width 0.25) (layer "F.Cu") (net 14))
 (segment (start 151.950872 89.720872) (end 151.950872 85.184128) (width 0.25) (layer "F.Cu") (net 14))
 (segment (start 153.473372 91.243372) (end 151.950872 89.720872) (width 0.25) (layer "F.Cu") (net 14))
 (segment (start 150.933372 91.243372) (end 149.180872 89.490872) (width 0.25) (layer "F.Cu") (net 15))
 (segment (start 150.933372 94.704128) (end 150.933372 91.243372) (width 0.25) (layer "F.Cu") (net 15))
 (segment (start 149.180872 89.490872) (end 149.180872 85.184128) (width 0.25) (layer "F.Cu") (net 15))
 (segment (start 148.393372 94.704128) (end 148.393372 91.243372) (width 0.25) (layer "F.Cu") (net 16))
 (segment (start 148.393372 91.243372) (end 146.410872 89.260872) (width 0.25) (layer "F.Cu") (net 16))
 (segment (start 146.410872 89.260872) (end 146.410872 85.184128) (width 0.25) (layer "F.Cu") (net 16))
 (segment (start 144.166333 84.436333) (end 144.166333 93.017089) (width 0.25) (layer "F.Cu") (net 7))
 (segment (start 145.025872 83.576794) (end 145.025872 82.344128) (width 0.25) (layer "F.Cu") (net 7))
 (segment (start 144.166333 84.436333) (end 145.025872 83.576794) (width 0.25) (layer "F.Cu") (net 7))
 (segment (start 144.166333 93.017089) (end 145.853372 94.704128) (width 0.25) (layer "F.Cu") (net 7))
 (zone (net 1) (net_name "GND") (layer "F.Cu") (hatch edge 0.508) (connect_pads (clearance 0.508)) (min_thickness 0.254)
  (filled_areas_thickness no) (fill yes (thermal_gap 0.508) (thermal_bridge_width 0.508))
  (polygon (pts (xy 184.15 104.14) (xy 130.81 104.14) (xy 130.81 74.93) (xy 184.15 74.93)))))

